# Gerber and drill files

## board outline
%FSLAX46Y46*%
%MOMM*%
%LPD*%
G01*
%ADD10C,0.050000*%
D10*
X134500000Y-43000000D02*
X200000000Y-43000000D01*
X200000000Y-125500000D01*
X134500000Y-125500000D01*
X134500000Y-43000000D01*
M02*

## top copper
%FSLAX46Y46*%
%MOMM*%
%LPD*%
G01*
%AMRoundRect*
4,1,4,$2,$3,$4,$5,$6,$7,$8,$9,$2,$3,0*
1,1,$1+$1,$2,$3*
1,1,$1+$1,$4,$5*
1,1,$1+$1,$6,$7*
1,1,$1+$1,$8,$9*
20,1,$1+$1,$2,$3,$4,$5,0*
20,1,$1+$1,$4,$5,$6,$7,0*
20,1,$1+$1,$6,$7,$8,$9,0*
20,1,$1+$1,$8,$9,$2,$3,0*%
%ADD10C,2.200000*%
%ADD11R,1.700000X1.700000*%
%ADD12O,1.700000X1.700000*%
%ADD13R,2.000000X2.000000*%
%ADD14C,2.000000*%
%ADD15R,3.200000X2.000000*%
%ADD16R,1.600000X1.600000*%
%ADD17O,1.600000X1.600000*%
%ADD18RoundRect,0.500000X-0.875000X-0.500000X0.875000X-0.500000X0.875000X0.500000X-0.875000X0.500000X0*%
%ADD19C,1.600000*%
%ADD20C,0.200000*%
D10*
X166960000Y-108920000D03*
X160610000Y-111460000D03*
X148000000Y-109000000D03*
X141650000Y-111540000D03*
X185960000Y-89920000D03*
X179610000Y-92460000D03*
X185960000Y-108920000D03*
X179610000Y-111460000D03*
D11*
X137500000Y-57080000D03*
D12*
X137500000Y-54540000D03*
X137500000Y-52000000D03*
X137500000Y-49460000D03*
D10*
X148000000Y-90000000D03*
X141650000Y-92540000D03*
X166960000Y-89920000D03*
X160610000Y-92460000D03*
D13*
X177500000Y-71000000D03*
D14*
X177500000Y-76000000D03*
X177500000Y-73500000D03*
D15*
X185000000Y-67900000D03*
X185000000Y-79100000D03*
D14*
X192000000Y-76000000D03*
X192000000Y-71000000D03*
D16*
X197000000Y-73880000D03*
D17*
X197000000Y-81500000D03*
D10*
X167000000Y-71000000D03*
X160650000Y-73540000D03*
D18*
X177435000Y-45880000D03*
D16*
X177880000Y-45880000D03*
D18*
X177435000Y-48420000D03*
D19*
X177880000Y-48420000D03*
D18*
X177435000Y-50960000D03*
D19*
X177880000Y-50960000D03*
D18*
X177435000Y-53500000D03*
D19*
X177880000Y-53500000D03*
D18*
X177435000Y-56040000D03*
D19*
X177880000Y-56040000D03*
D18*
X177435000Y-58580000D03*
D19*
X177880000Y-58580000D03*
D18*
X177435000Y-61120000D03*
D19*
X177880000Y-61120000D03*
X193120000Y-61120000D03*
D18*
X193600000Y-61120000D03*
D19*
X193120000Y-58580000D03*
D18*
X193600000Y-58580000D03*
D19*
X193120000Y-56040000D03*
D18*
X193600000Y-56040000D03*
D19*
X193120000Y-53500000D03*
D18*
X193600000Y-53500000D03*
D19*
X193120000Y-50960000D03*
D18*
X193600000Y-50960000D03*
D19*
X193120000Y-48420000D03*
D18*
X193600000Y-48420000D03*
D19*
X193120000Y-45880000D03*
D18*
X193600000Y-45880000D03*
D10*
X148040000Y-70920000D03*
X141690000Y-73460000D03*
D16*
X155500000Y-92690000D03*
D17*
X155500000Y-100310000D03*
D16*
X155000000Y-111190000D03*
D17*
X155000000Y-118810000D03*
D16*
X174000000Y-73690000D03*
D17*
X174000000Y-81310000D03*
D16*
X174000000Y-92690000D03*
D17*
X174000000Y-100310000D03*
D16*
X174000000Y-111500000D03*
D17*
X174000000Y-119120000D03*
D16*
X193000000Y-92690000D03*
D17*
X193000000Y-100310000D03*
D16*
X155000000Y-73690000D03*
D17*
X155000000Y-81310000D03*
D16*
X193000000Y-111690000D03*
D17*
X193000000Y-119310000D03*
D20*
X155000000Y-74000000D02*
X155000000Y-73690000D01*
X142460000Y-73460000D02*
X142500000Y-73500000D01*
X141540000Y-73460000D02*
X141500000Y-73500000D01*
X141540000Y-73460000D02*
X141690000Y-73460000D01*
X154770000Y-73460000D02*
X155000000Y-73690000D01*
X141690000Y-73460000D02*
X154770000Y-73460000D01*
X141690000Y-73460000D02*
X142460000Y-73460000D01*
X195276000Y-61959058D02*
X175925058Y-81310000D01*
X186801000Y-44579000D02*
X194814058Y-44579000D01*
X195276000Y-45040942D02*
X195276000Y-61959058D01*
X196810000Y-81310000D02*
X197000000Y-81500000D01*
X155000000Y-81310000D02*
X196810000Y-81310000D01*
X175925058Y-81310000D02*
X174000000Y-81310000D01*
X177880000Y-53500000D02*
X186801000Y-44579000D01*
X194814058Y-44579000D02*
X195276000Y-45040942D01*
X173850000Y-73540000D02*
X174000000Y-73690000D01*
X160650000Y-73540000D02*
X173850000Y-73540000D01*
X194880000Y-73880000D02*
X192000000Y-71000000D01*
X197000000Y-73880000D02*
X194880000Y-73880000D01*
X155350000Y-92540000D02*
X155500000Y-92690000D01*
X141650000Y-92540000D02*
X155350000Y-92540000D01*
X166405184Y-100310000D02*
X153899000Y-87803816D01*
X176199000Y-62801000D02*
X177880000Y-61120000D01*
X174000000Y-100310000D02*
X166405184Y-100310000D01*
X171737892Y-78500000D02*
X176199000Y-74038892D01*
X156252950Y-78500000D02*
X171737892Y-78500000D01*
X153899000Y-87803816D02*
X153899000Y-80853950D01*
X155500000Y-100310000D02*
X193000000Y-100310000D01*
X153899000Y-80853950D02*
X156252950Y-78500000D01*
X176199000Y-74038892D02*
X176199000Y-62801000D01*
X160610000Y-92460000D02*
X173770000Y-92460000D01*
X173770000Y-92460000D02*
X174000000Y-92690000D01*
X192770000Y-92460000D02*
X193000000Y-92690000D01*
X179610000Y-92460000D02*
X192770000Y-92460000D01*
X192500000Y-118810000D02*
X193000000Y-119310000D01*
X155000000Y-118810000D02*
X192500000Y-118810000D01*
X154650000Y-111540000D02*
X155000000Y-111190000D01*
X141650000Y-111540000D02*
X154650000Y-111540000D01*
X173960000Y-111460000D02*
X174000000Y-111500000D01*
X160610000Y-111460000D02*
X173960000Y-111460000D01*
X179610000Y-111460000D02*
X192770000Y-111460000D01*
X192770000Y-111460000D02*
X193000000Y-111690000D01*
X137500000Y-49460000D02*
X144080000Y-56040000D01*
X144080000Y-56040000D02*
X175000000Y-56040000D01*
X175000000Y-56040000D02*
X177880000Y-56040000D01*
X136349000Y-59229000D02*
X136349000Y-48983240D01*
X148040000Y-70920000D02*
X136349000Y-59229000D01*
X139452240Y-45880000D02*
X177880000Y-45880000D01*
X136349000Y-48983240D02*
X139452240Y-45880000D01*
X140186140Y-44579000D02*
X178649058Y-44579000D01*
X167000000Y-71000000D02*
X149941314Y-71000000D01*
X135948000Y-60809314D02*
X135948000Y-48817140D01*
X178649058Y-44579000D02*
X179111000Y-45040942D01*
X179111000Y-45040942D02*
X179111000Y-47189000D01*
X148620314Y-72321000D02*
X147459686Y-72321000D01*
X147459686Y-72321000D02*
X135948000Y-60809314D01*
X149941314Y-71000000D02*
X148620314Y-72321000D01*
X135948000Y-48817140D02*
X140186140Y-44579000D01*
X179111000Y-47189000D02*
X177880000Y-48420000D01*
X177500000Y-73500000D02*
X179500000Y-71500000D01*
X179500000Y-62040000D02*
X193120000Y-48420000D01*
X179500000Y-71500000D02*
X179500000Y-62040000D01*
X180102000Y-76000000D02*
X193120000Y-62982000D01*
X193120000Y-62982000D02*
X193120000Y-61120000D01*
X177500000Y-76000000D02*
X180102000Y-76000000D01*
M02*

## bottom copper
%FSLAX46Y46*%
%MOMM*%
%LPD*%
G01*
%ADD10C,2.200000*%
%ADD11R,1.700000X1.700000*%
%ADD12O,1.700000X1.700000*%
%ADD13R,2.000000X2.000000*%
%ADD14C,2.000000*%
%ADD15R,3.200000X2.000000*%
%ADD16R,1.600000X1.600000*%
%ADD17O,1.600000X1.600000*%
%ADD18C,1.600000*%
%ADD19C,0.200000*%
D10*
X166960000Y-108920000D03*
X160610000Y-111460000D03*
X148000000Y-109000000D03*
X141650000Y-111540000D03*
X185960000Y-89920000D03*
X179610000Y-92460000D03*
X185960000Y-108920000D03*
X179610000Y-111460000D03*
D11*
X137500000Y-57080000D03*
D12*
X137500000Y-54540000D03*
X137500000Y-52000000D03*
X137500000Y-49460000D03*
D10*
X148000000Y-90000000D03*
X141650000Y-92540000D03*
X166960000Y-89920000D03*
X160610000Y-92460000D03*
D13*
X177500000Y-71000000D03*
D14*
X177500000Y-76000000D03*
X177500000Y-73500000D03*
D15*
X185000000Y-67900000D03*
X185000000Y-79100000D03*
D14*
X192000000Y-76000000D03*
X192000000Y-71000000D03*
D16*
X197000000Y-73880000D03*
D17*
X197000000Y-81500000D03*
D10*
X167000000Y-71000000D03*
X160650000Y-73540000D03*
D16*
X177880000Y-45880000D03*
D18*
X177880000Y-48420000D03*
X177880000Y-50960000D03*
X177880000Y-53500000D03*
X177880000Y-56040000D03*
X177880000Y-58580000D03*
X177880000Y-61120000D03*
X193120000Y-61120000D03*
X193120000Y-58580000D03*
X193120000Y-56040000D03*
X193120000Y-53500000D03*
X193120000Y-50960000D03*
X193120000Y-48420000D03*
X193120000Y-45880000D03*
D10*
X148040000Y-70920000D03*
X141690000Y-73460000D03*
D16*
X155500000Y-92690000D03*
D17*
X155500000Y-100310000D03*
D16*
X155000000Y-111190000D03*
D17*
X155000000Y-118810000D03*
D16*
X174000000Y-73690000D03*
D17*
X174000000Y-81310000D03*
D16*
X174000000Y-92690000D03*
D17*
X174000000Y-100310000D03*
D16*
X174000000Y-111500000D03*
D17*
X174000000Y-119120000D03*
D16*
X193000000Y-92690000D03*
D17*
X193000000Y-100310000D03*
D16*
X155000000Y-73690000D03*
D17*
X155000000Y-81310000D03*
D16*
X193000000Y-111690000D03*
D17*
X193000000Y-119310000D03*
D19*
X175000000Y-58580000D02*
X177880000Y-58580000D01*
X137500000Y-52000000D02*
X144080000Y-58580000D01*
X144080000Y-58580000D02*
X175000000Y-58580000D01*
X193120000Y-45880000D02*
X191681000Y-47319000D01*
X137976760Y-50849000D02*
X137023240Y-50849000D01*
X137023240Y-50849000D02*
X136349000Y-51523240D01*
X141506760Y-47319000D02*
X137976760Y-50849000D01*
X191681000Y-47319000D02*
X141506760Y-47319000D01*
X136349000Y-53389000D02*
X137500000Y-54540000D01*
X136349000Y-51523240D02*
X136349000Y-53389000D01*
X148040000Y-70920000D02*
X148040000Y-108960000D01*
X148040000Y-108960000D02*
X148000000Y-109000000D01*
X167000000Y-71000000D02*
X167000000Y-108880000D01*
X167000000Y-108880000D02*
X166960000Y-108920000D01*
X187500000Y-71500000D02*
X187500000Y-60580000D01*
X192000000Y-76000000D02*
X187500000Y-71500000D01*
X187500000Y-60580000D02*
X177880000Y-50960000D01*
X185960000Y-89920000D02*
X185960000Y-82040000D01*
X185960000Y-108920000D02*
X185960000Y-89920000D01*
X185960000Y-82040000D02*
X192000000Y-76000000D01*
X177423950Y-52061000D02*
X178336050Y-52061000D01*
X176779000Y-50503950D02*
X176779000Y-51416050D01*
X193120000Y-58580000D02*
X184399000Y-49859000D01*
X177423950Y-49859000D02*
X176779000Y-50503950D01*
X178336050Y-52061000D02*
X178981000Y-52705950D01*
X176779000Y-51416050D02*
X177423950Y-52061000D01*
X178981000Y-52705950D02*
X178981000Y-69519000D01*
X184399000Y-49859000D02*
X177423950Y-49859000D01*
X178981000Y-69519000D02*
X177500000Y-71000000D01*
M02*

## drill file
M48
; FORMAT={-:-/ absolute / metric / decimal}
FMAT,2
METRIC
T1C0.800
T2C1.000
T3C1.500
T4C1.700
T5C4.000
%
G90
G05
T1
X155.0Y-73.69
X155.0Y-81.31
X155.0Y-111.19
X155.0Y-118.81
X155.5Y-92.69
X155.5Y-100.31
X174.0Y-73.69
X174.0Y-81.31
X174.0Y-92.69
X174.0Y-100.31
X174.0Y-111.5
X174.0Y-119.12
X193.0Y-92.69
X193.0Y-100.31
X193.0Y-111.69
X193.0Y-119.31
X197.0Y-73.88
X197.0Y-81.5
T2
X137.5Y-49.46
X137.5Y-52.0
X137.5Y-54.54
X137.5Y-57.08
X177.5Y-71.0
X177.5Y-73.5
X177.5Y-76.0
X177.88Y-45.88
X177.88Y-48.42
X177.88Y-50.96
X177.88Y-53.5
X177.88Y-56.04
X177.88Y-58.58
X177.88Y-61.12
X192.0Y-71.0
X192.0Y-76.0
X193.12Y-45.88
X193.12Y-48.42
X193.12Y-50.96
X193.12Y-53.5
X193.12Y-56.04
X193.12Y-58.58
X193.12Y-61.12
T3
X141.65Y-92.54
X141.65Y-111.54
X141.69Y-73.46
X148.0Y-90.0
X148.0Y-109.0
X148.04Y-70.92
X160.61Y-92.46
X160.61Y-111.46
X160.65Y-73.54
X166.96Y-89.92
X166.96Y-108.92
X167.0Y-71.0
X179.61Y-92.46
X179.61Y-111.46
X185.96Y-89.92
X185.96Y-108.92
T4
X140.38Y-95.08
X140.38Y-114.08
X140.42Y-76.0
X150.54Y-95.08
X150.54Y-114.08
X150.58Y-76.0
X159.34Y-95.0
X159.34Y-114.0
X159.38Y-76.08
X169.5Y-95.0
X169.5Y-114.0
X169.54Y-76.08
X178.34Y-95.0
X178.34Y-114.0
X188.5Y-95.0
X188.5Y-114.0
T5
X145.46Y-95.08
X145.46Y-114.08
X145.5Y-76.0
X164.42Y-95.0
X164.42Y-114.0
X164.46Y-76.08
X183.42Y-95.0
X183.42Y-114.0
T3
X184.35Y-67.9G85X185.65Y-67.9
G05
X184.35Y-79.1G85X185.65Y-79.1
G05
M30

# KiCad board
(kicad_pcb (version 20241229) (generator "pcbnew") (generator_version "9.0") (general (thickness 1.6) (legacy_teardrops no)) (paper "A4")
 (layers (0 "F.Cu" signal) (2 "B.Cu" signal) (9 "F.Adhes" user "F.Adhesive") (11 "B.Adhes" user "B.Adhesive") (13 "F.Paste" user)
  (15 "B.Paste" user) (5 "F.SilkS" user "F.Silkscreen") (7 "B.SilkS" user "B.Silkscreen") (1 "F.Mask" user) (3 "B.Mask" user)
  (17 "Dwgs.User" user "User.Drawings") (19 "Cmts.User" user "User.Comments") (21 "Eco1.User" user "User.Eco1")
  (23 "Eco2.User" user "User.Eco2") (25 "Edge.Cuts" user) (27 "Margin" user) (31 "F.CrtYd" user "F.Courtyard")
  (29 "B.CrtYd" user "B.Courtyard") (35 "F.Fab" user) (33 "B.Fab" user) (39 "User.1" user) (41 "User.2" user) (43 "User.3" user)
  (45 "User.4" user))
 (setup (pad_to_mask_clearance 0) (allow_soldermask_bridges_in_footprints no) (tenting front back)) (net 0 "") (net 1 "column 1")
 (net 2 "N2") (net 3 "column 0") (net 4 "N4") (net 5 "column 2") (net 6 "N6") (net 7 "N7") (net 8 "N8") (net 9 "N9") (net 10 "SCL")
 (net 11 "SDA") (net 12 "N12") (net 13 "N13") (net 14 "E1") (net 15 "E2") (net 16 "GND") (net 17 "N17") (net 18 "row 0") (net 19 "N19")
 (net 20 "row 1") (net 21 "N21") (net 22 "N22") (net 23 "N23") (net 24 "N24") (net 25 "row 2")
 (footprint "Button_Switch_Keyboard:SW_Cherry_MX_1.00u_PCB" (layer "F.Cu") (at 166.96 108.92)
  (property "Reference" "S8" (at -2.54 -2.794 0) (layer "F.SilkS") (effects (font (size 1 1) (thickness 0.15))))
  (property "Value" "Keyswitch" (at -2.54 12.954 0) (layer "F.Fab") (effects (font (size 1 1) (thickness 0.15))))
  (pad "" np_thru_hole circle (at -7.62 5.08) (size 1.7 1.7) (drill 1.7) (layers "*.Cu" "*.Mask"))
  (pad "" np_thru_hole circle (at -2.54 5.08) (size 4 4) (drill 4) (layers "*.Cu" "*.Mask"))
  (pad "" np_thru_hole circle (at 2.54 5.08) (size 1.7 1.7) (drill 1.7) (layers "*.Cu" "*.Mask"))
  (pad "1" thru_hole circle (at 0 0) (size 2.2 2.2) (drill 1.5) (layers "*.Cu" "*.Mask") (remove_unused_layers no) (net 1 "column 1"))
  (pad "2" thru_hole circle (at -6.35 2.54) (size 2.2 2.2) (drill 1.5) (layers "*.Cu" "*.Mask") (remove_unused_layers no) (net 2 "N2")))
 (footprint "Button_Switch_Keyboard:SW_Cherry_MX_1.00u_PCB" (layer "F.Cu") (at 148 109)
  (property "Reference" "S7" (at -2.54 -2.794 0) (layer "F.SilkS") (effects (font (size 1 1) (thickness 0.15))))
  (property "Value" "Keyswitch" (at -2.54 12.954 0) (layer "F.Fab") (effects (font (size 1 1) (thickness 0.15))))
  (pad "" np_thru_hole circle (at -7.62 5.08) (size 1.7 1.7) (drill 1.7) (layers "*.Cu" "*.Mask"))
  (pad "" np_thru_hole circle (at -2.54 5.08) (size 4 4) (drill 4) (layers "*.Cu" "*.Mask"))
  (pad "" np_thru_hole circle (at 2.54 5.08) (size 1.7 1.7) (drill 1.7) (layers "*.Cu" "*.Mask"))
  (pad "1" thru_hole circle (at 0 0) (size 2.2 2.2) (drill 1.5) (layers "*.Cu" "*.Mask") (remove_unused_layers no) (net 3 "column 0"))
  (pad "2" thru_hole circle (at -6.35 2.54) (size 2.2 2.2) (drill 1.5) (layers "*.Cu" "*.Mask") (remove_unused_layers no) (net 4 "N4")))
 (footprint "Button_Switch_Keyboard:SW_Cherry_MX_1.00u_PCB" (layer "F.Cu") (at 185.96 89.92)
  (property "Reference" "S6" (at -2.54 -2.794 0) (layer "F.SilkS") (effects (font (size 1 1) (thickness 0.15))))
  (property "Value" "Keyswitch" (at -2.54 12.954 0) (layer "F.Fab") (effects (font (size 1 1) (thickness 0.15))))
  (pad "" np_thru_hole circle (at -7.62 5.08) (size 1.7 1.7) (drill 1.7) (layers "*.Cu" "*.Mask"))
  (pad "" np_thru_hole circle (at -2.54 5.08) (size 4 4) (drill 4) (layers "*.Cu" "*.Mask"))
  (pad "" np_thru_hole circle (at 2.54 5.08) (size 1.7 1.7) (drill 1.7) (layers "*.Cu" "*.Mask"))
  (pad "1" thru_hole circle (at 0 0) (size 2.2 2.2) (drill 1.5) (layers "*.Cu" "*.Mask") (remove_unused_layers no) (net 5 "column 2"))
  (pad "2" thru_hole circle (at -6.35 2.54) (size 2.2 2.2) (drill 1.5) (layers "*.Cu" "*.Mask") (remove_unused_layers no) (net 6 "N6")))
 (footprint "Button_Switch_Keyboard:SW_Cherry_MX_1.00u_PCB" (layer "F.Cu") (at 185.96 108.92)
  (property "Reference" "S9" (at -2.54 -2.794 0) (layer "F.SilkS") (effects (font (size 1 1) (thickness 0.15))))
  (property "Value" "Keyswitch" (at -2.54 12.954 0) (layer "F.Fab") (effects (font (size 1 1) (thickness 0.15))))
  (pad "" np_thru_hole circle (at -7.62 5.08) (size 1.7 1.7) (drill 1.7) (layers "*.Cu" "*.Mask"))
  (pad "" np_thru_hole circle (at -2.54 5.08) (size 4 4) (drill 4) (layers "*.Cu" "*.Mask"))
  (pad "" np_thru_hole circle (at 2.54 5.08) (size 1.7 1.7) (drill 1.7) (layers "*.Cu" "*.Mask"))
  (pad "1" thru_hole circle (at 0 0) (size 2.2 2.2) (drill 1.5) (layers "*.Cu" "*.Mask") (remove_unused_layers no) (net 5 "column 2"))
  (pad "2" thru_hole circle (at -6.35 2.54) (size 2.2 2.2) (drill 1.5) (layers "*.Cu" "*.Mask") (remove_unused_layers no) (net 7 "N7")))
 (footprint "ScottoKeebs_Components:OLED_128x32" (layer "F.Cu") (at 135.9 47.28)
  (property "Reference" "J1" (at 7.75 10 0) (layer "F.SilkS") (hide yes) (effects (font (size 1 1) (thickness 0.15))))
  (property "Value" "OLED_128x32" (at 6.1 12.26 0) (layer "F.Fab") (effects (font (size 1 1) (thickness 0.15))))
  (pad "1" thru_hole rect (at 1.6 9.8 180) (size 1.7 1.7) (drill 1) (layers "*.Cu" "*.Mask") (remove_unused_layers no) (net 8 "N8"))
  (pad "2" thru_hole oval (at 1.6 7.26 180) (size 1.7 1.7) (drill 1) (layers "*.Cu" "*.Mask") (remove_unused_layers no) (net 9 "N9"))
  (pad "3" thru_hole oval (at 1.6 4.72 180) (size 1.7 1.7) (drill 1) (layers "*.Cu" "*.Mask") (remove_unused_layers no) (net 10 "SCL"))
  (pad "4" thru_hole oval (at 1.6 2.18 180) (size 1.7 1.7) (drill 1) (layers "*.Cu" "*.Mask") (remove_unused_layers no) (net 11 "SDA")))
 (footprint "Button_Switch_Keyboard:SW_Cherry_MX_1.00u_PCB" (layer "F.Cu") (at 148 90)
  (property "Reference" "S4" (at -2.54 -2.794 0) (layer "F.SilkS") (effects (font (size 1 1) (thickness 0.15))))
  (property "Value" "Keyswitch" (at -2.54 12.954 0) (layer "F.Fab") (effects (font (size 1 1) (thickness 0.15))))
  (pad "" np_thru_hole circle (at -7.62 5.08) (size 1.7 1.7) (drill 1.7) (layers "*.Cu" "*.Mask"))
  (pad "" np_thru_hole circle (at -2.54 5.08) (size 4 4) (drill 4) (layers "*.Cu" "*.Mask"))
  (pad "" np_thru_hole circle (at 2.54 5.08) (size 1.7 1.7) (drill 1.7) (layers "*.Cu" "*.Mask"))
  (pad "1" thru_hole circle (at 0 0) (size 2.2 2.2) (drill 1.5) (layers "*.Cu" "*.Mask") (remove_unused_layers no) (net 3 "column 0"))
  (pad "2" thru_hole circle (at -6.35 2.54) (size 2.2 2.2) (drill 1.5) (layers "*.Cu" "*.Mask") (remove_unused_layers no) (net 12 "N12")))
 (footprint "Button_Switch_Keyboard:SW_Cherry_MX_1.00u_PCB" (layer "F.Cu") (at 166.96 89.92)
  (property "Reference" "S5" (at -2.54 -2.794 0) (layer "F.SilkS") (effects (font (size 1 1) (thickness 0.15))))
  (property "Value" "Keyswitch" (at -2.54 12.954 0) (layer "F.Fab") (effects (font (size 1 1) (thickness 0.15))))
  (pad "" np_thru_hole circle (at -7.62 5.08) (size 1.7 1.7) (drill 1.7) (layers "*.Cu" "*.Mask"))
  (pad "" np_thru_hole circle (at -2.54 5.08) (size 4 4) (drill 4) (layers "*.Cu" "*.Mask"))
  (pad "" np_thru_hole circle (at 2.54 5.08) (size 1.7 1.7) (drill 1.7) (layers "*.Cu" "*.Mask"))
  (pad "1" thru_hole circle (at 0 0) (size 2.2 2.2) (drill 1.5) (layers "*.Cu" "*.Mask") (remove_unused_layers no) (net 1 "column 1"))
  (pad "2" thru_hole circle (at -6.35 2.54) (size 2.2 2.2) (drill 1.5) (layers "*.Cu" "*.Mask") (remove_unused_layers no) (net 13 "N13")))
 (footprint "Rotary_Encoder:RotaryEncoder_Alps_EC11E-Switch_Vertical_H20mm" (layer "F.Cu") (at 177.5 71)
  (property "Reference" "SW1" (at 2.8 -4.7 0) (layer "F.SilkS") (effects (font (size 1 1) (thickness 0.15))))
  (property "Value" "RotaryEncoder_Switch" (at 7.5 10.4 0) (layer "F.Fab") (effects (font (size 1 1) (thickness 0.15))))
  (pad "A" thru_hole rect (at 0 0) (size 2 2) (drill 1) (layers "*.Cu" "*.Mask") (remove_unused_layers no) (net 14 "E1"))
  (pad "B" thru_hole circle (at 0 5) (size 2 2) (drill 1) (layers "*.Cu" "*.Mask") (remove_unused_layers no) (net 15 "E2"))
  (pad "C" thru_hole circle (at 0 2.5) (size 2 2) (drill 1) (layers "*.Cu" "*.Mask") (remove_unused_layers no) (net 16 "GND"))
  (pad "MP" thru_hole rect (at 7.5 -3.1) (size 3.2 2) (drill oval 2.8 1.5) (layers "*.Cu" "*.Mask") (remove_unused_layers no))
  (pad "MP" thru_hole rect (at 7.5 8.1) (size 3.2 2) (drill oval 2.8 1.5) (layers "*.Cu" "*.Mask") (remove_unused_layers no))
  (pad "S1" thru_hole circle (at 14.5 5) (size 2 2) (drill 1) (layers "*.Cu" "*.Mask") (remove_unused_layers no) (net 5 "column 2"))
  (pad "S2" thru_hole circle (at 14.5 0) (size 2 2) (drill 1) (layers "*.Cu" "*.Mask") (remove_unused_layers no) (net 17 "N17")))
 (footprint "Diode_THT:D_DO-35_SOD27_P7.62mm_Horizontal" (layer "F.Cu") (at 197 73.88 -90)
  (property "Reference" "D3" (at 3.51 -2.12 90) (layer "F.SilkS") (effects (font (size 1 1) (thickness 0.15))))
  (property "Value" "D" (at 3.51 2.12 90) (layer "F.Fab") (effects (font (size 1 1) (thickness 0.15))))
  (pad "1" thru_hole rect (at 0 0 270) (size 1.6 1.6) (drill 0.8) (layers "*.Cu" "*.Mask") (remove_unused_layers no) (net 17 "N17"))
  (pad "2" thru_hole oval (at 7.62 0 270) (size 1.6 1.6) (drill 0.8) (layers "*.Cu" "*.Mask") (remove_unused_layers no) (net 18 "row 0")))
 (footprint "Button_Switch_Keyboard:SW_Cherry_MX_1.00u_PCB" (layer "F.Cu") (at 167 71)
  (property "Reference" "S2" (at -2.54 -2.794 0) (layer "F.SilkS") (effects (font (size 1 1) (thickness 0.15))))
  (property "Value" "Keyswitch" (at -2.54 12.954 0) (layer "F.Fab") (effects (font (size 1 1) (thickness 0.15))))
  (pad "" np_thru_hole circle (at -7.62 5.08) (size 1.7 1.7) (drill 1.7) (layers "*.Cu" "*.Mask"))
  (pad "" np_thru_hole circle (at -2.54 5.08) (size 4 4) (drill 4) (layers "*.Cu" "*.Mask"))
  (pad "" np_thru_hole circle (at 2.54 5.08) (size 1.7 1.7) (drill 1.7) (layers "*.Cu" "*.Mask"))
  (pad "1" thru_hole circle (at 0 0) (size 2.2 2.2) (drill 1.5) (layers "*.Cu" "*.Mask") (remove_unused_layers no) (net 1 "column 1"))
  (pad "2" thru_hole circle (at -6.35 2.54) (size 2.2 2.2) (drill 1.5) (layers "*.Cu" "*.Mask") (remove_unused_layers no) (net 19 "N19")))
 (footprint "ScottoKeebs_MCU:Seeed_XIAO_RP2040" (layer "F.Cu") (at 185.5 53.5)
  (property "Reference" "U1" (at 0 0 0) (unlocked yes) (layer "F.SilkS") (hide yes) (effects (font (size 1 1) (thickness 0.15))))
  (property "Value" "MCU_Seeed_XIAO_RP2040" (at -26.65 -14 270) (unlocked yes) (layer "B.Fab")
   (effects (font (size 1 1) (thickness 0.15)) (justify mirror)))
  (pad "1" smd roundrect (at -8.065 -7.62) (size 2.75 2) (layers "F.Cu" "F.Mask" "F.Paste") (roundrect_rratio 0.25) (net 3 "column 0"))
  (pad "1" thru_hole rect (at -7.62 -7.62 90) (size 1.6 1.6) (drill 1) (layers "*.Cu" "*.Mask") (remove_unused_layers no) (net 3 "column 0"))
  (pad "2" smd roundrect (at -8.065 -5.08) (size 2.75 2) (layers "F.Cu" "F.Mask" "F.Paste") (roundrect_rratio 0.25) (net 1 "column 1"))
  (pad "2" thru_hole circle (at -7.62 -5.08 90) (size 1.6 1.6) (drill 1) (layers "*.Cu" "*.Mask") (remove_unused_layers no)
   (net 1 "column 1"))
  (pad "3" smd roundrect (at -8.065 -2.54) (size 2.75 2) (layers "F.Cu" "F.Mask" "F.Paste") (roundrect_rratio 0.25) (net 5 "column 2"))
  (pad "3" thru_hole circle (at -7.62 -2.54 90) (size 1.6 1.6) (drill 1) (layers "*.Cu" "*.Mask") (remove_unused_layers no)
   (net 5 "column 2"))
  (pad "4" smd roundrect (at -8.065 0) (size 2.75 2) (layers "F.Cu" "F.Mask" "F.Paste") (roundrect_rratio 0.25) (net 18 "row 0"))
  (pad "4" thru_hole circle (at -7.62 0 90) (size 1.6 1.6) (drill 1) (layers "*.Cu" "*.Mask") (remove_unused_layers no) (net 18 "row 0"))
  (pad "5" smd roundrect (at -8.065 2.54) (size 2.75 2) (layers "F.Cu" "F.Mask" "F.Paste") (roundrect_rratio 0.25) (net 11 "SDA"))
  (pad "5" thru_hole circle (at -7.62 2.54 90) (size 1.6 1.6) (drill 1) (layers "*.Cu" "*.Mask") (remove_unused_layers no) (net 11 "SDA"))
  (pad "6" smd roundrect (at -8.065 5.08) (size 2.75 2) (layers "F.Cu" "F.Mask" "F.Paste") (roundrect_rratio 0.25) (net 10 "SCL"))
  (pad "6" thru_hole circle (at -7.62 5.08 90) (size 1.6 1.6) (drill 1) (layers "*.Cu" "*.Mask") (remove_unused_layers no) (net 10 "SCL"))
  (pad "7" smd roundrect (at -8.065 7.62) (size 2.75 2) (layers "F.Cu" "F.Mask" "F.Paste") (roundrect_rratio 0.25) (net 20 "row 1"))
  (pad "7" thru_hole circle (at -7.62 7.62 90) (size 1.6 1.6) (drill 1) (layers "*.Cu" "*.Mask") (remove_unused_layers no) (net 20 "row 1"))
  (pad "8" thru_hole circle (at 7.62 7.62 90) (size 1.6 1.6) (drill 1) (layers "*.Cu" "*.Mask") (remove_unused_layers no) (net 15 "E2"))
  (pad "8" smd roundrect (at 8.1 7.62) (size 2.75 2) (layers "F.Cu" "F.Mask" "F.Paste") (roundrect_rratio 0.25) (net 15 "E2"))
  (pad "9" thru_hole circle (at 7.62 5.08 90) (size 1.6 1.6) (drill 1) (layers "*.Cu" "*.Mask") (remove_unused_layers no) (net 14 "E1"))
  (pad "9" smd roundrect (at 8.1 5.08) (size 2.75 2) (layers "F.Cu" "F.Mask" "F.Paste") (roundrect_rratio 0.25) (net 14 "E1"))
  (pad "10" thru_hole circle (at 7.62 2.54 90) (size 1.6 1.6) (drill 1) (layers "*.Cu" "*.Mask") (remove_unused_layers no) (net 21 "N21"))
  (pad "10" smd roundrect (at 8.1 2.54) (size 2.75 2) (layers "F.Cu" "F.Mask" "F.Paste") (roundrect_rratio 0.25) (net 21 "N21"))
  (pad "11" thru_hole circle (at 7.62 0 90) (size 1.6 1.6) (drill 1) (layers "*.Cu" "*.Mask") (remove_unused_layers no) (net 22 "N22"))
  (pad "11" smd roundrect (at 8.1 0) (size 2.75 2) (layers "F.Cu" "F.Mask" "F.Paste") (roundrect_rratio 0.25) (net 22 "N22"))
  (pad "12" thru_hole circle (at 7.62 -2.54 90) (size 1.6 1.6) (drill 1) (layers "*.Cu" "*.Mask") (remove_unused_layers no) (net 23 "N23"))
  (pad "12" smd roundrect (at 8.1 -2.54) (size 2.75 2) (layers "F.Cu" "F.Mask" "F.Paste") (roundrect_rratio 0.25) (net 23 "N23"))
  (pad "13" thru_hole circle (at 7.62 -5.08 90) (size 1.6 1.6) (drill 1) (layers "*.Cu" "*.Mask") (remove_unused_layers no) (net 16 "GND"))
  (pad "13" smd roundrect (at 8.1 -5.08) (size 2.75 2) (layers "F.Cu" "F.Mask" "F.Paste") (roundrect_rratio 0.25) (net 16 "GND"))
  (pad "14" thru_hole circle (at 7.62 -7.62 90) (size 1.6 1.6) (drill 1) (layers "*.Cu" "*.Mask") (remove_unused_layers no) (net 9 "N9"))
  (pad "14" smd roundrect (at 8.1 -7.62) (size 2.75 2) (layers "F.Cu" "F.Mask" "F.Paste") (roundrect_rratio 0.25) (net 9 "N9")))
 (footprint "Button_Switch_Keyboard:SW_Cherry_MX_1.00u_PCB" (layer "F.Cu") (at 148.04 70.92)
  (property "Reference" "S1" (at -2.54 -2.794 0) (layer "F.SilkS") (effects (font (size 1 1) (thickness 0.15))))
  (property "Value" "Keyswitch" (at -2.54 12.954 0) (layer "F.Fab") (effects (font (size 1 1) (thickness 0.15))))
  (pad "" np_thru_hole circle (at -7.62 5.08) (size 1.7 1.7) (drill 1.7) (layers "*.Cu" "*.Mask"))
  (pad "" np_thru_hole circle (at -2.54 5.08) (size 4 4) (drill 4) (layers "*.Cu" "*.Mask"))
  (pad "" np_thru_hole circle (at 2.54 5.08) (size 1.7 1.7) (drill 1.7) (layers "*.Cu" "*.Mask"))
  (pad "1" thru_hole circle (at 0 0) (size 2.2 2.2) (drill 1.5) (layers "*.Cu" "*.Mask") (remove_unused_layers no) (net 3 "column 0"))
  (pad "2" thru_hole circle (at -6.35 2.54) (size 2.2 2.2) (drill 1.5) (layers "*.Cu" "*.Mask") (remove_unused_layers no) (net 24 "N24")))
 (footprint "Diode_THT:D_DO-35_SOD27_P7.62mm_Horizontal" (layer "B.Cu") (at 155.5 92.69 -90)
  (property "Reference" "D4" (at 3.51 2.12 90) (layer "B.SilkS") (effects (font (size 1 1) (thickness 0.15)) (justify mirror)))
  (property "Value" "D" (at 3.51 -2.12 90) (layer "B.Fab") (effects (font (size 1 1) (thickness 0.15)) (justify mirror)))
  (pad "1" thru_hole rect (at 0 0 270) (size 1.6 1.6) (drill 0.8) (layers "*.Cu" "*.Mask") (remove_unused_layers no) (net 12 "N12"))
  (pad "2" thru_hole oval (at 7.62 0 270) (size 1.6 1.6) (drill 0.8) (layers "*.Cu" "*.Mask") (remove_unused_layers no) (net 20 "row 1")))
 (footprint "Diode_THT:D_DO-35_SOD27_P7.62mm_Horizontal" (layer "B.Cu") (at 155 111.19 -90)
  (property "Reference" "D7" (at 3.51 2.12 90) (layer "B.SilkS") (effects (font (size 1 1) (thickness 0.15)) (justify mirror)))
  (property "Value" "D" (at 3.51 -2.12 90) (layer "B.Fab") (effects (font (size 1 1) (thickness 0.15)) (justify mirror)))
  (pad "1" thru_hole rect (at 0 0 270) (size 1.6 1.6) (drill 0.8) (layers "*.Cu" "*.Mask") (remove_unused_layers no) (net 4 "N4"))
  (pad "2" thru_hole oval (at 7.62 0 270) (size 1.6 1.6) (drill 0.8) (layers "*.Cu" "*.Mask") (remove_unused_layers no) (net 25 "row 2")))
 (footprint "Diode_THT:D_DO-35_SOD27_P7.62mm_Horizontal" (layer "B.Cu") (at 174 73.69 -90)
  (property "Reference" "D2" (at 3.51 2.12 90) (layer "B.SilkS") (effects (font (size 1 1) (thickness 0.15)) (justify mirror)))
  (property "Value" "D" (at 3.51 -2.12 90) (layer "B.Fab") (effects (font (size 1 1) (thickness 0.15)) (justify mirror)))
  (pad "1" thru_hole rect (at 0 0 270) (size 1.6 1.6) (drill 0.8) (layers "*.Cu" "*.Mask") (remove_unused_layers no) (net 19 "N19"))
  (pad "2" thru_hole oval (at 7.62 0 270) (size 1.6 1.6) (drill 0.8) (layers "*.Cu" "*.Mask") (remove_unused_layers no) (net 18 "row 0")))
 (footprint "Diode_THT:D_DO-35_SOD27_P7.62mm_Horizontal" (layer "B.Cu") (at 174 92.69 -90)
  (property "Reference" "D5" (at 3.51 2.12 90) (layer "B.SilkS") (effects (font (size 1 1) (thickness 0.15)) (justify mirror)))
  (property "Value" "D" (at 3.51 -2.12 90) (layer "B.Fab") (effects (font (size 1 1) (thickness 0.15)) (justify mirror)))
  (pad "1" thru_hole rect (at 0 0 270) (size 1.6 1.6) (drill 0.8) (layers "*.Cu" "*.Mask") (remove_unused_layers no) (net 13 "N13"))
  (pad "2" thru_hole oval (at 7.62 0 270) (size 1.6 1.6) (drill 0.8) (layers "*.Cu" "*.Mask") (remove_unused_layers no) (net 20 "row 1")))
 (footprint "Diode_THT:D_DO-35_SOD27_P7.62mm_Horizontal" (layer "B.Cu") (at 174 111.5 -90)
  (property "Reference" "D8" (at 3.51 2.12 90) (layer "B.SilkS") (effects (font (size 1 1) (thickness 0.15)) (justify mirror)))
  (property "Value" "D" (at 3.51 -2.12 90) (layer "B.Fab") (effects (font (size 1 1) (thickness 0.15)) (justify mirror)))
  (pad "1" thru_hole rect (at 0 0 270) (size 1.6 1.6) (drill 0.8) (layers "*.Cu" "*.Mask") (remove_unused_layers no) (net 2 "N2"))
  (pad "2" thru_hole oval (at 7.62 0 270) (size 1.6 1.6) (drill 0.8) (layers "*.Cu" "*.Mask") (remove_unused_layers no) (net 25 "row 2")))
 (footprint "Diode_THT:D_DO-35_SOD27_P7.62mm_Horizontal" (layer "B.Cu") (at 193 92.69 -90)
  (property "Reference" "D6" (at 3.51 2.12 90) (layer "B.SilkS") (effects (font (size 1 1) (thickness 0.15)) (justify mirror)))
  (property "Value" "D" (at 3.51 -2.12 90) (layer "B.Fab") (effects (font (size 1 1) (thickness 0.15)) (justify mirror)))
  (pad "1" thru_hole rect (at 0 0 270) (size 1.6 1.6) (drill 0.8) (layers "*.Cu" "*.Mask") (remove_unused_layers no) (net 6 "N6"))
  (pad "2" thru_hole oval (at 7.62 0 270) (size 1.6 1.6) (drill 0.8) (layers "*.Cu" "*.Mask") (remove_unused_layers no) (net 20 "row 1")))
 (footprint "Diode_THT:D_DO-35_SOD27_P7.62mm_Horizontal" (layer "B.Cu") (at 155 73.69 -90)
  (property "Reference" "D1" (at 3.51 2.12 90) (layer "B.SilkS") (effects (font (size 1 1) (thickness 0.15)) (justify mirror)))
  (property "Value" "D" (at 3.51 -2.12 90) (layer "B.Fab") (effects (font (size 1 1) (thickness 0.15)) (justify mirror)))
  (pad "1" thru_hole rect (at 0 0 270) (size 1.6 1.6) (drill 0.8) (layers "*.Cu" "*.Mask") (remove_unused_layers no) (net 24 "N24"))
  (pad "2" thru_hole oval (at 7.62 0 270) (size 1.6 1.6) (drill 0.8) (layers "*.Cu" "*.Mask") (remove_unused_layers no) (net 18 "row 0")))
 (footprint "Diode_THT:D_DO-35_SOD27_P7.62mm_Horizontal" (layer "B.Cu") (at 193 111.69 -90)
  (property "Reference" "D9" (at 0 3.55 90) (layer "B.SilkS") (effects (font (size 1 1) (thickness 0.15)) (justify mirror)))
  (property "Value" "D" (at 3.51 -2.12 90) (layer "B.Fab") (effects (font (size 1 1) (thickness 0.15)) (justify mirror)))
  (pad "1" thru_hole rect (at 0 0 270) (size 1.6 1.6) (drill 0.8) (layers "*.Cu" "*.Mask") (remove_unused_layers no) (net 7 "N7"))
  (pad "2" thru_hole oval (at 7.62 0 270) (size 1.6 1.6) (drill 0.8) (layers "*.Cu" "*.Mask") (remove_unused_layers no) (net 25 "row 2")))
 (gr_rect (start 134.5 43) (end 200 125.5) (stroke (width 0.05) (type default)) (fill no) (layer "Edge.Cuts"))
 (segment (start 155 74) (end 155 73.69) (width 0.2) (layer "F.Cu") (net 24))
 (segment (start 142.46 73.46) (end 142.5 73.5) (width 0.2) (layer "F.Cu") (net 24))
 (segment (start 141.54 73.46) (end 141.5 73.5) (width 0.2) (layer "F.Cu") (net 24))
 (segment (start 141.54 73.46) (end 141.69 73.46) (width 0.2) (layer "F.Cu") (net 24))
 (segment (start 154.77 73.46) (end 155 73.69) (width 0.2) (layer "F.Cu") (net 24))
 (segment (start 141.69 73.46) (end 154.77 73.46) (width 0.2) (layer "F.Cu") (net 24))
 (segment (start 141.69 73.46) (end 142.46 73.46) (width 0.2) (layer "F.Cu") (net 24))
 (segment (start 195.276 61.959058) (end 175.925058 81.31) (width 0.2) (layer "F.Cu") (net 18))
 (segment (start 186.801 44.579) (end 194.814058 44.579) (width 0.2) (layer "F.Cu") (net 18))
 (segment (start 195.276 45.040942) (end 195.276 61.959058) (width 0.2) (layer "F.Cu") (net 18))
 (segment (start 196.81 81.31) (end 197 81.5) (width 0.2) (layer "F.Cu") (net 18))
 (segment (start 155 81.31) (end 196.81 81.31) (width 0.2) (layer "F.Cu") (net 18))
 (segment (start 175.925058 81.31) (end 174 81.31) (width 0.2) (layer "F.Cu") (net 18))
 (segment (start 177.88 53.5) (end 186.801 44.579) (width 0.2) (layer "F.Cu") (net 18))
 (segment (start 194.814058 44.579) (end 195.276 45.040942) (width 0.2) (layer "F.Cu") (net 18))
 (segment (start 173.85 73.54) (end 174 73.69) (width 0.2) (layer "F.Cu") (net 19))
 (segment (start 160.65 73.54) (end 173.85 73.54) (width 0.2) (layer "F.Cu") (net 19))
 (segment (start 194.88 73.88) (end 192 71) (width 0.2) (layer "F.Cu") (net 17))
 (segment (start 197 73.88) (end 194.88 73.88) (width 0.2) (layer "F.Cu") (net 17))
 (segment (start 155.35 92.54) (end 155.5 92.69) (width 0.2) (layer "F.Cu") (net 12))
 (segment (start 141.65 92.54) (end 155.35 92.54) (width 0.2) (layer "F.Cu") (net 12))
 (segment (start 166.405184 100.31) (end 153.899 87.803816) (width 0.2) (layer "F.Cu") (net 20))
 (segment (start 176.199 62.801) (end 177.88 61.12) (width 0.2) (layer "F.Cu") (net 20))
 (segment (start 174 100.31) (end 166.405184 100.31) (width 0.2) (layer "F.Cu") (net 20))
 (segment (start 171.737892 78.5) (end 176.199 74.038892) (width 0.2) (layer "F.Cu") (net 20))
 (segment (start 156.25295 78.5) (end 171.737892 78.5) (width 0.2) (layer "F.Cu") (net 20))
 (segment (start 153.899 87.803816) (end 153.899 80.85395) (width 0.2) (layer "F.Cu") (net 20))
 (segment (start 155.5 100.31) (end 193 100.31) (width 0.2) (layer "F.Cu") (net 20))
 (segment (start 153.899 80.85395) (end 156.25295 78.5) (width 0.2) (layer "F.Cu") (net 20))
 (segment (start 176.199 74.038892) (end 176.199 62.801) (width 0.2) (layer "F.Cu") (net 20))
 (segment (start 160.61 92.46) (end 173.77 92.46) (width 0.2) (layer "F.Cu") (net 13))
 (segment (start 173.77 92.46) (end 174 92.69) (width 0.2) (layer "F.Cu") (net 13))
 (segment (start 192.77 92.46) (end 193 92.69) (width 0.2) (layer "F.Cu") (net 6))
 (segment (start 179.61 92.46) (end 192.77 92.46) (width 0.2) (layer "F.Cu") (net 6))
 (segment (start 192.5 118.81) (end 193 119.31) (width 0.2) (layer "F.Cu") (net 25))
 (segment (start 155 118.81) (end 192.5 118.81) (width 0.2) (layer "F.Cu") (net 25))
 (segment (start 154.65 111.54) (end 155 111.19) (width 0.2) (layer "F.Cu") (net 4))
 (segment (start 141.65 111.54) (end 154.65 111.54) (width 0.2) (layer "F.Cu") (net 4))
 (segment (start 173.96 111.46) (end 174 111.5) (width 0.2) (layer "F.Cu") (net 2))
 (segment (start 160.61 111.46) (end 173.96 111.46) (width 0.2) (layer "F.Cu") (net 2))
 (segment (start 179.61 111.46) (end 192.77 111.46) (width 0.2) (layer "F.Cu") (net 7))
 (segment (start 192.77 111.46) (end 193 111.69) (width 0.2) (layer "F.Cu") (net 7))
 (segment (start 175 58.58) (end 177.88 58.58) (width 0.2) (layer "B.Cu") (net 10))
 (segment (start 137.5 52) (end 144.08 58.58) (width 0.2) (layer "B.Cu") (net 10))
 (segment (start 144.08 58.58) (end 175 58.58) (width 0.2) (layer "B.Cu") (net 10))
 (segment (start 137.5 49.46) (end 144.08 56.04) (width 0.2) (layer "F.Cu") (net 11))
 (segment (start 144.08 56.04) (end 175 56.04) (width 0.2) (layer "F.Cu") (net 11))
 (segment (start 175 56.04) (end 177.88 56.04) (width 0.2) (layer "F.Cu") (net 11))
 (segment (start 193.12 45.88) (end 191.681 47.319) (width 0.2) (layer "B.Cu") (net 9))
 (segment (start 137.97676 50.849) (end 137.02324 50.849) (width 0.2) (layer "B.Cu") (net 9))
 (segment (start 137.02324 50.849) (end 136.349 51.52324) (width 0.2) (layer "B.Cu") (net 9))
 (segment (start 141.50676 47.319) (end 137.97676 50.849) (width 0.2) (layer "B.Cu") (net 9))
 (segment (start 191.681 47.319) (end 141.50676 47.319) (width 0.2) (layer "B.Cu") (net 9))
 (segment (start 136.349 53.389) (end 137.5 54.54) (width 0.2) (layer "B.Cu") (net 9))
 (segment (start 136.349 51.52324) (end 136.349 53.389) (width 0.2) (layer "B.Cu") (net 9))
 (segment (start 136.349 59.229) (end 136.349 48.98324) (width 0.2) (layer "F.Cu") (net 3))
 (segment (start 148.04 70.92) (end 136.349 59.229) (width 0.2) (layer "F.Cu") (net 3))
 (segment (start 139.45224 45.88) (end 177.88 45.88) (width 0.2) (layer "F.Cu") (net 3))
 (segment (start 136.349 48.98324) (end 139.45224 45.88) (width 0.2) (layer "F.Cu") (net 3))
 (segment (start 148.04 70.92) (end 148.04 108.96) (width 0.2) (layer "B.Cu") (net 3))
 (segment (start 148.04 108.96) (end 148 109) (width 0.2) (layer "B.Cu") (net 3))
 (segment (start 140.18614 44.579) (end 178.649058 44.579) (width 0.2) (layer "F.Cu") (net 1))
 (segment (start 167 71) (end 149.941314 71) (width 0.2) (layer "F.Cu") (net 1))
 (segment (start 135.948 60.809314) (end 135.948 48.81714) (width 0.2) (layer "F.Cu") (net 1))
 (segment (start 178.649058 44.579) (end 179.111 45.040942) (width 0.2) (layer "F.Cu") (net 1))
 (segment (start 179.111 45.040942) (end 179.111 47.189) (width 0.2) (layer "F.Cu") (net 1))
 (segment (start 148.620314 72.321) (end 147.459686 72.321) (width 0.2) (layer "F.Cu") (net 1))
 (segment (start 147.459686 72.321) (end 135.948 60.809314) (width 0.2) (layer "F.Cu") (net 1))
 (segment (start 149.941314 71) (end 148.620314 72.321) (width 0.2) (layer "F.Cu") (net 1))
 (segment (start 135.948 48.81714) (end 140.18614 44.579) (width 0.2) (layer "F.Cu") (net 1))
 (segment (start 179.111 47.189) (end 177.88 48.42) (width 0.2) (layer "F.Cu") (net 1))
 (segment (start 167 71) (end 167 108.88) (width 0.2) (layer "B.Cu") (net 1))
 (segment (start 167 108.88) (end 166.96 108.92) (width 0.2) (layer "B.Cu") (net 1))
 (segment (start 187.5 71.5) (end 187.5 60.58) (width 0.2) (layer "B.Cu") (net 5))
 (segment (start 192 76) (end 187.5 71.5) (width 0.2) (layer "B.Cu") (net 5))
 (segment (start 187.5 60.58) (end 177.88 50.96) (width 0.2) (layer "B.Cu") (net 5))
 (segment (start 185.96 89.92) (end 185.96 82.04) (width 0.2) (layer "B.Cu") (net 5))
 (segment (start 185.96 108.92) (end 185.96 89.92) (width 0.2) (layer "B.Cu") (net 5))
 (segment (start 185.96 82.04) (end 192 76) (width 0.2) (layer "B.Cu") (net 5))
 (segment (start 177.5 73.5) (end 179.5 71.5) (width 0.2) (layer "F.Cu") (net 16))
 (segment (start 179.5 62.04) (end 193.12 48.42) (width 0.2) (layer "F.Cu") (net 16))
 (segment (start 179.5 71.5) (end 179.5 62.04) (width 0.2) (layer "F.Cu") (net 16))
 (segment (start 177.42395 52.061) (end 178.33605 52.061) (width 0.2) (layer "B.Cu") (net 14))
 (segment (start 176.779 50.50395) (end 176.779 51.41605) (width 0.2) (layer "B.Cu") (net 14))
 (segment (start 193.12 58.58) (end 184.399 49.859) (width 0.2) (layer "B.Cu") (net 14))
 (segment (start 177.42395 49.859) (end 176.779 50.50395) (width 0.2) (layer "B.Cu") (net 14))
 (segment (start 178.33605 52.061) (end 178.981 52.70595) (width 0.2) (layer "B.Cu") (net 14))
 (segment (start 176.779 51.41605) (end 177.42395 52.061) (width 0.2) (layer "B.Cu") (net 14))
 (segment (start 178.981 52.70595) (end 178.981 69.519) (width 0.2) (layer "B.Cu") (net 14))
 (segment (start 184.399 49.859) (end 177.42395 49.859) (width 0.2) (layer "B.Cu") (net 14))
 (segment (start 178.981 69.519) (end 177.5 71) (width 0.2) (layer "B.Cu") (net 14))
 (segment (start 180.102 76) (end 193.12 62.982) (width 0.2) (layer "F.Cu") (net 15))
 (segment (start 193.12 62.982) (end 193.12 61.12) (width 0.2) (layer "F.Cu") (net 15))
 (segment (start 177.5 76) (end 180.102 76) (width 0.2) (layer "F.Cu") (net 15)))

